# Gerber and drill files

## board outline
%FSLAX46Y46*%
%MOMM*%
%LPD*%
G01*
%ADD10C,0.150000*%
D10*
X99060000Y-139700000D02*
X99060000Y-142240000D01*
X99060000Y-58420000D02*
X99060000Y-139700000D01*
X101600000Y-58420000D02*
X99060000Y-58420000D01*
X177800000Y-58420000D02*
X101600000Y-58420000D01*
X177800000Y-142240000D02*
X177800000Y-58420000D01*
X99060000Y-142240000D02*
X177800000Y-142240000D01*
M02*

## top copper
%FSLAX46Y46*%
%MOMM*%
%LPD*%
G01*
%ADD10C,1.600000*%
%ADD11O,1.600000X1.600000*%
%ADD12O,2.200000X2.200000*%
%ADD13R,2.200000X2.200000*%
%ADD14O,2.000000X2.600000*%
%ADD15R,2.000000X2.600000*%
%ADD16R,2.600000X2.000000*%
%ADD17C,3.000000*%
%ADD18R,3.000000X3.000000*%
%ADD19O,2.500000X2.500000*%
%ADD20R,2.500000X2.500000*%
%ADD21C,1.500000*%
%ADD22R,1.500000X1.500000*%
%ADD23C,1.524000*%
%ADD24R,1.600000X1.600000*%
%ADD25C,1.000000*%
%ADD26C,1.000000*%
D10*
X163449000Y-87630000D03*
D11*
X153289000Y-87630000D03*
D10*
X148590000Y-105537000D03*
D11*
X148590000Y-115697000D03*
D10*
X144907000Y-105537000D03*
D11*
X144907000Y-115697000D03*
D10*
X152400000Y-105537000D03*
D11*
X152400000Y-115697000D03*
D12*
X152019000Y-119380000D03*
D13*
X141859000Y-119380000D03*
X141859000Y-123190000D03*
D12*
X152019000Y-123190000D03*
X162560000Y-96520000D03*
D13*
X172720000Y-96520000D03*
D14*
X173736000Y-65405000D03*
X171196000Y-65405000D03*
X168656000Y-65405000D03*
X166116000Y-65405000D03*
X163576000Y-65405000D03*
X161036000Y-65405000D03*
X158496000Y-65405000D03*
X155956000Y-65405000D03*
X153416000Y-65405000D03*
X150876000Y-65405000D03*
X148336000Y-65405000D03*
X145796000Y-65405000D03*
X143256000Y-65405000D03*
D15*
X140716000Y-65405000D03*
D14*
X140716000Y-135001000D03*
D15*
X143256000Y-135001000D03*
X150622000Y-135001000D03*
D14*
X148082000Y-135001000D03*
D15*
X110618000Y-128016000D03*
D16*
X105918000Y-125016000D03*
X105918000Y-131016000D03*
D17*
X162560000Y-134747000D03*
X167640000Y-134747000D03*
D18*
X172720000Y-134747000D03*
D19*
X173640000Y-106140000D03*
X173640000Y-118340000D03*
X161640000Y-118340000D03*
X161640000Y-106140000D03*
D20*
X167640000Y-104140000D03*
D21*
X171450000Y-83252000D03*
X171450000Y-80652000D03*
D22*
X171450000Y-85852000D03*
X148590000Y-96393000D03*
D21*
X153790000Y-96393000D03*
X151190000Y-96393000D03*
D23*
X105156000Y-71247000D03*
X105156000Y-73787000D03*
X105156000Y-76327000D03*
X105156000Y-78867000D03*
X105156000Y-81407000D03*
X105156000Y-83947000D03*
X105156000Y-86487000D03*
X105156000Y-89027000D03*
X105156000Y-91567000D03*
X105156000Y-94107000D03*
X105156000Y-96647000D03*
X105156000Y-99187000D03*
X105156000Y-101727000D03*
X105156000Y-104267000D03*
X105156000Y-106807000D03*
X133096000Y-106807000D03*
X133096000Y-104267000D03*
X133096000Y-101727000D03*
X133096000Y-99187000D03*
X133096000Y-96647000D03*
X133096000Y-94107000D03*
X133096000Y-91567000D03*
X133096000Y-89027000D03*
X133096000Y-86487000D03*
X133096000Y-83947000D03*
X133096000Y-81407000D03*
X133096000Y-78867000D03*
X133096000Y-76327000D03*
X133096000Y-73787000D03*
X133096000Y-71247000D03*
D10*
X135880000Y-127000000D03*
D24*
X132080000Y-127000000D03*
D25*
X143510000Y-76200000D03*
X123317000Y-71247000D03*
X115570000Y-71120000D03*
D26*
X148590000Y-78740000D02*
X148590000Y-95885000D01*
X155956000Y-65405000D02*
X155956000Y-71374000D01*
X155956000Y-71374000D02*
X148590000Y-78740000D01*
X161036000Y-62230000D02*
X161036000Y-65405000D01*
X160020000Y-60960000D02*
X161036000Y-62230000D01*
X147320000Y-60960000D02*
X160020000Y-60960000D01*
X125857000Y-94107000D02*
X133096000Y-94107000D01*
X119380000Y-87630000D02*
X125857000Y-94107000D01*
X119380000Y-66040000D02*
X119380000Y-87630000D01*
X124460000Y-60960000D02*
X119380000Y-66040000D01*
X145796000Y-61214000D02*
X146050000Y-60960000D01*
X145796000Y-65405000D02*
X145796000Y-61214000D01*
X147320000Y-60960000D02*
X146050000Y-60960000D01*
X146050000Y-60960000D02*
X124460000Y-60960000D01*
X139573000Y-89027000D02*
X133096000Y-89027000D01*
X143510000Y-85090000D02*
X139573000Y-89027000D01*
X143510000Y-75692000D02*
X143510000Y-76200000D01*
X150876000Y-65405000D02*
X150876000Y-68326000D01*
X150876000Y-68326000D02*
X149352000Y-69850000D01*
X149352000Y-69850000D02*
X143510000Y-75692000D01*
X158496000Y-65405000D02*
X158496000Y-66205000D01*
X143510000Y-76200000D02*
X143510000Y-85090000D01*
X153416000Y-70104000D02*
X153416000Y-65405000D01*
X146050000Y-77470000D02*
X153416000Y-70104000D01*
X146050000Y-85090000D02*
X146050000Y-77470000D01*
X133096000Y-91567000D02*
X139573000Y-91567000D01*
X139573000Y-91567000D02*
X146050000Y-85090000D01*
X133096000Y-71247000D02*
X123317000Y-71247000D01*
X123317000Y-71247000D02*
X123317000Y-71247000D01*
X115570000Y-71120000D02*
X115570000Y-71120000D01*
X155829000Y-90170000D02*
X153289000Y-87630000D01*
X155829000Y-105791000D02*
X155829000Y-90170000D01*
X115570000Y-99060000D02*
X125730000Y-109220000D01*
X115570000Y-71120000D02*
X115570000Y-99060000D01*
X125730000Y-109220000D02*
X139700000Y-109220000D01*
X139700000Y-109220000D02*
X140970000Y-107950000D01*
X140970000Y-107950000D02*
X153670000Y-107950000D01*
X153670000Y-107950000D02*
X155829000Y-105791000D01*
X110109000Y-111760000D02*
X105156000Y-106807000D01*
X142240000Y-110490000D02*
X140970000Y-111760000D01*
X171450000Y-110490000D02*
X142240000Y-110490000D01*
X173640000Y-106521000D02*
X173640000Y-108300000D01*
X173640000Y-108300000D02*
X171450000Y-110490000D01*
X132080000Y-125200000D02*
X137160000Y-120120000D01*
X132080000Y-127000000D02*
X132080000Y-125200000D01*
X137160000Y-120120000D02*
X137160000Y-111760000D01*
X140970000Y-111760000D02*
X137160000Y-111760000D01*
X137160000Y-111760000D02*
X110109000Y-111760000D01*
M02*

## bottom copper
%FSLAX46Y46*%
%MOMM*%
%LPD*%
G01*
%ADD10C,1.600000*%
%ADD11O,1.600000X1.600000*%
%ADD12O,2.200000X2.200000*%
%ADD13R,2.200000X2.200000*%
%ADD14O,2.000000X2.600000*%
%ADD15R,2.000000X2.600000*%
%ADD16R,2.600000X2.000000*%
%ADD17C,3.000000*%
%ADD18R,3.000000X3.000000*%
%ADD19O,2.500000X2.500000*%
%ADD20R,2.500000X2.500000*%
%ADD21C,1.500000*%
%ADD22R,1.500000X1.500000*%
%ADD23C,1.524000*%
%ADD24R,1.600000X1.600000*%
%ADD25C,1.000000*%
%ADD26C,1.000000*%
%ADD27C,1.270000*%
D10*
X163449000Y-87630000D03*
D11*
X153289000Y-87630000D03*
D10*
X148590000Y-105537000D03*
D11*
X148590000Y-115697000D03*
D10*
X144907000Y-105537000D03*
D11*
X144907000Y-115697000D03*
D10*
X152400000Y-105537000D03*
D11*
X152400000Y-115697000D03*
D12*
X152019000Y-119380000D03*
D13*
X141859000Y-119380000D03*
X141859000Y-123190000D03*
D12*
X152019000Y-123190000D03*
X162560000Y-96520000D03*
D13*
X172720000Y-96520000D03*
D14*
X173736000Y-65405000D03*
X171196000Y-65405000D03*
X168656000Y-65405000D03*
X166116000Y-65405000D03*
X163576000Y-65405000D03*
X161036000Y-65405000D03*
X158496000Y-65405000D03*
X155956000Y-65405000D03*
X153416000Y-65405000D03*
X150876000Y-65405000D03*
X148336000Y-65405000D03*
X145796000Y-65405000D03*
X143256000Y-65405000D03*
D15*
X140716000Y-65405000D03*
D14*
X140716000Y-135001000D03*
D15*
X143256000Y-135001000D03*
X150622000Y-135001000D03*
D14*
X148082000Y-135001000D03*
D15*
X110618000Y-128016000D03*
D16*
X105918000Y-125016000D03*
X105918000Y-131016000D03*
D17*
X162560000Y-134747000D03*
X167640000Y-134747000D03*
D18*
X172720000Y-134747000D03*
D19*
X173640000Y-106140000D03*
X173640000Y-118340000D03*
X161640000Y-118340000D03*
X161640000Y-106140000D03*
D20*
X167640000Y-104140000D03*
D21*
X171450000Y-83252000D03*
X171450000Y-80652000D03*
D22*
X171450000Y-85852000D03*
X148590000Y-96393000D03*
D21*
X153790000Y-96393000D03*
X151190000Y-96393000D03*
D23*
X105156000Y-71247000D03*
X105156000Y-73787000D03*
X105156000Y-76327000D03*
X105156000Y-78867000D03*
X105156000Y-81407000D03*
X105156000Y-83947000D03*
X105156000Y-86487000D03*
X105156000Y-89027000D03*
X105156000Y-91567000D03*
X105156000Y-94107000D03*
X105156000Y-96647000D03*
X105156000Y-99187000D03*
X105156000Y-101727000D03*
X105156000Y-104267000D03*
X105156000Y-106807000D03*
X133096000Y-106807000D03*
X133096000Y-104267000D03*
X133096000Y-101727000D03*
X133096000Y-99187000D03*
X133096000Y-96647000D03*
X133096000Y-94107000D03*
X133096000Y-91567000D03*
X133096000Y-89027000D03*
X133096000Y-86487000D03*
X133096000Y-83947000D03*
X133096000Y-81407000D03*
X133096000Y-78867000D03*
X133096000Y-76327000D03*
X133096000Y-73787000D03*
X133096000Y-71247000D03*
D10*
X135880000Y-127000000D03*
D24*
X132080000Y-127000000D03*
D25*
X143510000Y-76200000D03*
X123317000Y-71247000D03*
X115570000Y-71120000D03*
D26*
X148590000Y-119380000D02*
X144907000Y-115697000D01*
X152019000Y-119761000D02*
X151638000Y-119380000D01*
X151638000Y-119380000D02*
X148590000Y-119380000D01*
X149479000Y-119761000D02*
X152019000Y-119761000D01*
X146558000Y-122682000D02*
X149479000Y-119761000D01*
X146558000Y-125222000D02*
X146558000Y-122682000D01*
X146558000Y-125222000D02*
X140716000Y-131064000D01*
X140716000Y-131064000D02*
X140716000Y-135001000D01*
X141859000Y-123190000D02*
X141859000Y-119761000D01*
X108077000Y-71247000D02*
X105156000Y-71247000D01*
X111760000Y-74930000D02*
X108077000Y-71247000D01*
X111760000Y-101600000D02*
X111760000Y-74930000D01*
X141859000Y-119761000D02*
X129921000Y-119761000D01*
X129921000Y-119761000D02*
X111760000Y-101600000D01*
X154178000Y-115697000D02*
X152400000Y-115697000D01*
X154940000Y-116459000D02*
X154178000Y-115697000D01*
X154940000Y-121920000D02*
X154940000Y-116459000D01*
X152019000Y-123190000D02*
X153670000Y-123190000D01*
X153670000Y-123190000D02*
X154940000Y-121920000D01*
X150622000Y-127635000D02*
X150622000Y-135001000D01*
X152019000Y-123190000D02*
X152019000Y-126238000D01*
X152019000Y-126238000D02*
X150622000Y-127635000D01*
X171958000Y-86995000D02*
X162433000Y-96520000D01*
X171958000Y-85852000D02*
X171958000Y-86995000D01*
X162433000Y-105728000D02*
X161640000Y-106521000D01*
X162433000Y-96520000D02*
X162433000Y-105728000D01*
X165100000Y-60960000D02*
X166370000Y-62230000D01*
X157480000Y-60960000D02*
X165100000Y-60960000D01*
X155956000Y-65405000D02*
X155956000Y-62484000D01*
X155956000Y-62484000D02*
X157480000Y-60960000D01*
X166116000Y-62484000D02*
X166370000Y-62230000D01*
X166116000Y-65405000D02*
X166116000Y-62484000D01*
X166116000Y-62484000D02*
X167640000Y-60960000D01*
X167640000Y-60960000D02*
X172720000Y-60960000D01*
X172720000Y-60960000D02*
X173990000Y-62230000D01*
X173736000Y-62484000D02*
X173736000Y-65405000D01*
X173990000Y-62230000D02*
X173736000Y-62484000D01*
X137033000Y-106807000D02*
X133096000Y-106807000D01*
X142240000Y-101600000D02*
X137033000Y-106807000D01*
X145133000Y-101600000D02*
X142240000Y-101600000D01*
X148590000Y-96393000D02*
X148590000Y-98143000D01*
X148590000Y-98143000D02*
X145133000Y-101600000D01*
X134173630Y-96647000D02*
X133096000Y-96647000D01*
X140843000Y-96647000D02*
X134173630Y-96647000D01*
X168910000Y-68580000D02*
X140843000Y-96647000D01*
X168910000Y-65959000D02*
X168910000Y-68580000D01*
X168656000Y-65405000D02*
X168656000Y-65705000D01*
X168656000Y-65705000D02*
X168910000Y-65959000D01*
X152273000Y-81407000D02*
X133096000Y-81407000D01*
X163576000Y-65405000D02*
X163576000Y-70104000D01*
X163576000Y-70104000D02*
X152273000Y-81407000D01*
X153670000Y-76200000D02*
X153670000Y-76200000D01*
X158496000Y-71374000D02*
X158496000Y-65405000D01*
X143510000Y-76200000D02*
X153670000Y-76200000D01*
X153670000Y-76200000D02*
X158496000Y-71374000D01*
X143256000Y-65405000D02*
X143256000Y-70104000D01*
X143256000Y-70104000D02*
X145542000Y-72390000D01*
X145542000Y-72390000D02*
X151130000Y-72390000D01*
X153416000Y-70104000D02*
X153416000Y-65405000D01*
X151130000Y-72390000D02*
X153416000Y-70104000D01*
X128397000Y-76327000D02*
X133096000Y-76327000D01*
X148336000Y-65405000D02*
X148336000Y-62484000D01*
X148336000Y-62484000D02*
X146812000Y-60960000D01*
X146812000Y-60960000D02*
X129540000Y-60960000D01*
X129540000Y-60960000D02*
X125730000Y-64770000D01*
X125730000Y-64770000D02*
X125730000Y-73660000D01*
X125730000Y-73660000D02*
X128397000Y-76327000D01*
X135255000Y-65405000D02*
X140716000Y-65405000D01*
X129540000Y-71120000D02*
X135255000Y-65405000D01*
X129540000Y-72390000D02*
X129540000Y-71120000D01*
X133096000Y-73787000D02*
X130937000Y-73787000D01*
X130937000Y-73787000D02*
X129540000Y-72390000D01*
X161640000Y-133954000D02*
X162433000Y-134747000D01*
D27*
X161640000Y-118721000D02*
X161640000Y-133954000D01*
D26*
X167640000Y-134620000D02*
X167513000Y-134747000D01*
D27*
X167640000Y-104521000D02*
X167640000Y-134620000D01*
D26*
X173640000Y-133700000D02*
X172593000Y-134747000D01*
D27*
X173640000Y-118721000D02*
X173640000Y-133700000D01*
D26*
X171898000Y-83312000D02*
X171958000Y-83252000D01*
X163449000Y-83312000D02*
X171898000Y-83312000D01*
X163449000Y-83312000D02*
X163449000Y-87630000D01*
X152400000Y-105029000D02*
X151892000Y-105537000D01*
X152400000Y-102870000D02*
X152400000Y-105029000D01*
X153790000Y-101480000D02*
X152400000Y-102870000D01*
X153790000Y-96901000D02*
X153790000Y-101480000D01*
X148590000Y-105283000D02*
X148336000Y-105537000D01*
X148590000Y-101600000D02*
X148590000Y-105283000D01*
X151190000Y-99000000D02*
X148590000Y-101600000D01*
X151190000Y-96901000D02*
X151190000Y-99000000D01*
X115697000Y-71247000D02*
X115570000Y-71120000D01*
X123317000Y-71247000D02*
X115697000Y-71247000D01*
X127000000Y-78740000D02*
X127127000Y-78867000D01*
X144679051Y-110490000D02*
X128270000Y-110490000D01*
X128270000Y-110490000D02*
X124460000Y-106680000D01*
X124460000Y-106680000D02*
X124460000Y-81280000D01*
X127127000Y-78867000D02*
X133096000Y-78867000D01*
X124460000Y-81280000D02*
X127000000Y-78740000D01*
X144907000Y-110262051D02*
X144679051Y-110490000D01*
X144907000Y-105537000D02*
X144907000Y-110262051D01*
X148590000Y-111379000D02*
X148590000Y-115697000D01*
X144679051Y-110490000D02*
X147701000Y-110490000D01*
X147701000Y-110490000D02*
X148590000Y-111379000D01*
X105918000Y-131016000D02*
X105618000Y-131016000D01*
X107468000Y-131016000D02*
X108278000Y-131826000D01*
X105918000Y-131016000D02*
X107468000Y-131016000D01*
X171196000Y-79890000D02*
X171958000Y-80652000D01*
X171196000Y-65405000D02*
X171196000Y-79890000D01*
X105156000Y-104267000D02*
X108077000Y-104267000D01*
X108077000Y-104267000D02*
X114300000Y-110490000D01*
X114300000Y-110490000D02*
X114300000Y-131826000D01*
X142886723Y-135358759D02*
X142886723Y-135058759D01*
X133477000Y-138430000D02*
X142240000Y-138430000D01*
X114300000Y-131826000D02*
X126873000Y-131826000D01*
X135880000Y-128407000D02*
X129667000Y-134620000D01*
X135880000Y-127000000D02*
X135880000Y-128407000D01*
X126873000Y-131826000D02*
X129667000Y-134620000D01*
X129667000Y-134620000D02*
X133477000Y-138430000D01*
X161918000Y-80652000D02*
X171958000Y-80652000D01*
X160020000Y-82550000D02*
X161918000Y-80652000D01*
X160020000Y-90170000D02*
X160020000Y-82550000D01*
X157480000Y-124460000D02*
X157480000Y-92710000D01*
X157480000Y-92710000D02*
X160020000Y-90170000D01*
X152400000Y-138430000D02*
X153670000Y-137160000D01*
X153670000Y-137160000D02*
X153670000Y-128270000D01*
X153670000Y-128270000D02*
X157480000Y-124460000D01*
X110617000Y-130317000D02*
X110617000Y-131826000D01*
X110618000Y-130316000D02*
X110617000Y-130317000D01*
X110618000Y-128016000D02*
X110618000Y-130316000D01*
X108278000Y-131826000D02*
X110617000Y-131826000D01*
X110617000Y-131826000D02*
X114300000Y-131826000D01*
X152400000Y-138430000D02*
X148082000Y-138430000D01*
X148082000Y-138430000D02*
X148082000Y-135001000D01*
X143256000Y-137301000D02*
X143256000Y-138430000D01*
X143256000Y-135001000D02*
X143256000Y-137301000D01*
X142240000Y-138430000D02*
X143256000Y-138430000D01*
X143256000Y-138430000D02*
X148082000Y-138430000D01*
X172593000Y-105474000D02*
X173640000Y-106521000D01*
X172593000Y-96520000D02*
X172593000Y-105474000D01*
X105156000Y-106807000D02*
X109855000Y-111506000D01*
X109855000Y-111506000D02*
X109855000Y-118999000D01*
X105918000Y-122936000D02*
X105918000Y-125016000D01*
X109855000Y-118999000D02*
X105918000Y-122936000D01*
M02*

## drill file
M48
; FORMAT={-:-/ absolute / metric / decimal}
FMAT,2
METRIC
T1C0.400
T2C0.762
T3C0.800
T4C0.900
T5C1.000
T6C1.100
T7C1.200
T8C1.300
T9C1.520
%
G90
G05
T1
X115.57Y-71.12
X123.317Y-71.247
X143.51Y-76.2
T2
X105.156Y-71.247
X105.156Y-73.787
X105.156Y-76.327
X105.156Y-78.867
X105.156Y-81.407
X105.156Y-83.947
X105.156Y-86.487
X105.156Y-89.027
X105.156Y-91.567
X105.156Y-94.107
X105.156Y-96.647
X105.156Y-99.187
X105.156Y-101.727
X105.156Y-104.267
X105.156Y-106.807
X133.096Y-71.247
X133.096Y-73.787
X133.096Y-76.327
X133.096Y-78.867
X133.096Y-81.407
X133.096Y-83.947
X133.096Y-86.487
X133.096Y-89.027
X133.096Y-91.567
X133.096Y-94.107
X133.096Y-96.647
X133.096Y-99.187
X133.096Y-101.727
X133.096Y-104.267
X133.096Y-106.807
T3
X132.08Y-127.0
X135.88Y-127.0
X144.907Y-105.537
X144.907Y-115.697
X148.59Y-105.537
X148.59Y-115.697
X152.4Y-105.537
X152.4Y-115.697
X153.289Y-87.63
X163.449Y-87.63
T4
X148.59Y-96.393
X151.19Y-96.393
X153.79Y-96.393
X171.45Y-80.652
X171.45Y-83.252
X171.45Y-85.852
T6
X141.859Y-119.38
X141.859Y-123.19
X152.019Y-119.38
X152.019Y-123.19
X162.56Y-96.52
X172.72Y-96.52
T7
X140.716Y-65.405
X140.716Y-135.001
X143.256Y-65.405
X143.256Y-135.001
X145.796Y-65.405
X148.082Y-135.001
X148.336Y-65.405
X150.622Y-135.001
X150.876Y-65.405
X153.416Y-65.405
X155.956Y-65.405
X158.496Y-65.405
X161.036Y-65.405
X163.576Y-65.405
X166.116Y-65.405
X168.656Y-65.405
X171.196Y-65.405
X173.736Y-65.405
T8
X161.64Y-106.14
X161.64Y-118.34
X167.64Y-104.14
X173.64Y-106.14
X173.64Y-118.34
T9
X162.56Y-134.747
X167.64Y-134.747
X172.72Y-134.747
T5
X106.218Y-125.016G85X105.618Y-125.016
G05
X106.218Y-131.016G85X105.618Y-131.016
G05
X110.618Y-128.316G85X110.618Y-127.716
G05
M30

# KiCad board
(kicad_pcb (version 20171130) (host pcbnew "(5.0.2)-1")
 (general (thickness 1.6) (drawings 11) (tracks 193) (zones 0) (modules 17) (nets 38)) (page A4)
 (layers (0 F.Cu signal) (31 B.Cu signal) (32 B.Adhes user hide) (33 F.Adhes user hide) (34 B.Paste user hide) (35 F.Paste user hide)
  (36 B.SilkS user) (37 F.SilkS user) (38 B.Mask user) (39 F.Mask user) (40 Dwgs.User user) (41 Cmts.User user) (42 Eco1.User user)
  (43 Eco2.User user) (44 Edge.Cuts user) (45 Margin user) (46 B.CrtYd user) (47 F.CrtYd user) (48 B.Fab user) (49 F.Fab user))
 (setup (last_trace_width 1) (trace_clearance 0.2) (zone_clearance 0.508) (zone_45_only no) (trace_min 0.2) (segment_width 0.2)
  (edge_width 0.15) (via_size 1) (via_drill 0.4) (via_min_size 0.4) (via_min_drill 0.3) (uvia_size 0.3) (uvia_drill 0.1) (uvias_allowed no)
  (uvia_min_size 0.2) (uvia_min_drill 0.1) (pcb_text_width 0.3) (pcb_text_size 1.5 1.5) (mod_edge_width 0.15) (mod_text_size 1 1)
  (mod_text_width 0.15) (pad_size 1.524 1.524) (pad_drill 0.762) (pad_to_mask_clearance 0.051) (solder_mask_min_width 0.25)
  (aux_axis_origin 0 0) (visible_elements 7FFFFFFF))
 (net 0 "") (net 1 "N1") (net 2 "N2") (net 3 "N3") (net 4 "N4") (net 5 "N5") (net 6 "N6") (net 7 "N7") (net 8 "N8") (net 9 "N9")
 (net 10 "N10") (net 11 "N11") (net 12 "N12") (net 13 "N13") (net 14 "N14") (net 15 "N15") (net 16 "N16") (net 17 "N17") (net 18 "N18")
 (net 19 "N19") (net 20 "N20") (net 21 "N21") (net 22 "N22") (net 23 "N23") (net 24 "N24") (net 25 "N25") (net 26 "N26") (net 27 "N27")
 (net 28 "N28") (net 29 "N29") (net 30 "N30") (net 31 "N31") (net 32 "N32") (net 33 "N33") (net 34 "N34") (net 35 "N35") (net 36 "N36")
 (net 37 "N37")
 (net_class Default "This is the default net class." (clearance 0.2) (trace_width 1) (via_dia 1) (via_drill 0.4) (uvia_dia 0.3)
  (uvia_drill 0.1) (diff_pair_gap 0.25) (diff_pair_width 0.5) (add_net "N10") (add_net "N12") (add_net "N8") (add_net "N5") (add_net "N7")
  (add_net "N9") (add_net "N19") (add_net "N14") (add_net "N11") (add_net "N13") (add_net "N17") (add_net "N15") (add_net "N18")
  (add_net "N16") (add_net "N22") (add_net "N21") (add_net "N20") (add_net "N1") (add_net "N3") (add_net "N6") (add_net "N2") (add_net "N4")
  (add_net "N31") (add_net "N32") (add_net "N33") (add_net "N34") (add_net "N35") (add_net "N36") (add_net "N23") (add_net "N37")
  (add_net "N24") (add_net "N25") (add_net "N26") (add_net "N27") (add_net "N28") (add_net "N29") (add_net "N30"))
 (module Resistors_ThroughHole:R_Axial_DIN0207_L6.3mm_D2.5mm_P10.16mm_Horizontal (layer F.Cu) (at 163.449 87.63 180)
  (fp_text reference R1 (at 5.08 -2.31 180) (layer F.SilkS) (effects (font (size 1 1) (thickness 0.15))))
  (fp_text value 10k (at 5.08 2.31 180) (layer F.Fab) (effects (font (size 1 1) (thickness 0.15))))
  (pad 1 thru_hole circle (at 0 0 180) (size 1.6 1.6) (drill 0.8) (layers *.Cu *.Mask) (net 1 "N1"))
  (pad 2 thru_hole oval (at 10.16 0 180) (size 1.6 1.6) (drill 0.8) (layers *.Cu *.Mask) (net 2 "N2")))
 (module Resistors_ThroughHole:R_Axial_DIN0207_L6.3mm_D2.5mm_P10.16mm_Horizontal (layer F.Cu) (at 148.59 105.537 270)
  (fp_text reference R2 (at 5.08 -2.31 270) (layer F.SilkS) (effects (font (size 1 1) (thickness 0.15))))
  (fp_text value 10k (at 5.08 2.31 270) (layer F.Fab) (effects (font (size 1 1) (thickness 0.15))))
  (pad 1 thru_hole circle (at 0 0 270) (size 1.6 1.6) (drill 0.8) (layers *.Cu *.Mask) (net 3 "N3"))
  (pad 2 thru_hole oval (at 10.16 0 270) (size 1.6 1.6) (drill 0.8) (layers *.Cu *.Mask) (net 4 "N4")))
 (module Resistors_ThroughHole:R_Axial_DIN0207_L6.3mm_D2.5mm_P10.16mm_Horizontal (layer F.Cu) (at 144.907 105.537 270)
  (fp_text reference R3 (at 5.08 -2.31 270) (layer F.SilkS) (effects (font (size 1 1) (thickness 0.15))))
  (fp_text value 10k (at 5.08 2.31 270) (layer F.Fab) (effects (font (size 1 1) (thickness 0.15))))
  (pad 1 thru_hole circle (at 0 0 270) (size 1.6 1.6) (drill 0.8) (layers *.Cu *.Mask) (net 4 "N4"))
  (pad 2 thru_hole oval (at 10.16 0 270) (size 1.6 1.6) (drill 0.8) (layers *.Cu *.Mask) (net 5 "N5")))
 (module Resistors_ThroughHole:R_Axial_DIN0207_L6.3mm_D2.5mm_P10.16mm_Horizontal (layer F.Cu) (at 152.4 105.537 270)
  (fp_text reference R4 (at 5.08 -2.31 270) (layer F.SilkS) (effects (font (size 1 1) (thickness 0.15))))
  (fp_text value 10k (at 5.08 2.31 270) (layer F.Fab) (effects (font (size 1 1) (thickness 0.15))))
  (pad 1 thru_hole circle (at 0 0 270) (size 1.6 1.6) (drill 0.8) (layers *.Cu *.Mask) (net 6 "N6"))
  (pad 2 thru_hole oval (at 10.16 0 270) (size 1.6 1.6) (drill 0.8) (layers *.Cu *.Mask) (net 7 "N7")))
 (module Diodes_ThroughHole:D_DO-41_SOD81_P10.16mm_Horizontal (layer F.Cu) (at 141.859 119.38)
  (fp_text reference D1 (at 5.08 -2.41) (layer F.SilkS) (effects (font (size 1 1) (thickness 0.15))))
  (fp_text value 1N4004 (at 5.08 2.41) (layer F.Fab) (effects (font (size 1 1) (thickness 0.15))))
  (pad 2 thru_hole oval (at 10.16 0) (size 2.2 2.2) (drill 1.1) (layers *.Cu *.Mask) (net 5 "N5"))
  (pad 1 thru_hole rect (at 0 0) (size 2.2 2.2) (drill 1.1) (layers *.Cu *.Mask) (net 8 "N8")))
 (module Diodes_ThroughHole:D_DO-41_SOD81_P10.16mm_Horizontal (layer F.Cu) (at 141.859 123.19)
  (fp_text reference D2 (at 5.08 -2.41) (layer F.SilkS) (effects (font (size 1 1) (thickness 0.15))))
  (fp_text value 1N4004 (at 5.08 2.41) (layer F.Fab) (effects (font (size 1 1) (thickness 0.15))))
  (pad 1 thru_hole rect (at 0 0) (size 2.2 2.2) (drill 1.1) (layers *.Cu *.Mask) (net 8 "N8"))
  (pad 2 thru_hole oval (at 10.16 0) (size 2.2 2.2) (drill 1.1) (layers *.Cu *.Mask) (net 7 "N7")))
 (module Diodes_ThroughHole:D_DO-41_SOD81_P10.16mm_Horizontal (layer F.Cu) (at 172.72 96.52 180)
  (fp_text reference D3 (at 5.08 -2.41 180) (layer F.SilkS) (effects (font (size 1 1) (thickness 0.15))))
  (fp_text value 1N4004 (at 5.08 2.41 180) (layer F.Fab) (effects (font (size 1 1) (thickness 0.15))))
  (pad 2 thru_hole oval (at 10.16 0 180) (size 2.2 2.2) (drill 1.1) (layers *.Cu *.Mask) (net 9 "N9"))
  (pad 1 thru_hole rect (at 0 0 180) (size 2.2 2.2) (drill 1.1) (layers *.Cu *.Mask) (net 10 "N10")))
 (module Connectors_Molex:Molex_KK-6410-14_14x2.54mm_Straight (layer F.Cu) (at 140.716 65.405)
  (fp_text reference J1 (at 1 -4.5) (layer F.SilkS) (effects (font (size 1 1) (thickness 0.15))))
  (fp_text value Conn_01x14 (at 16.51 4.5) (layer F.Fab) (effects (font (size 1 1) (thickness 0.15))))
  (pad 14 thru_hole oval (at 33.02 0) (size 2 2.6) (drill 1.2) (layers *.Cu *.Mask) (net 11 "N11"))
  (pad 13 thru_hole oval (at 30.48 0) (size 2 2.6) (drill 1.2) (layers *.Cu *.Mask) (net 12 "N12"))
  (pad 12 thru_hole oval (at 27.94 0) (size 2 2.6) (drill 1.2) (layers *.Cu *.Mask) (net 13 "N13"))
  (pad 11 thru_hole oval (at 25.4 0) (size 2 2.6) (drill 1.2) (layers *.Cu *.Mask) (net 11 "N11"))
  (pad 10 thru_hole oval (at 22.86 0) (size 2 2.6) (drill 1.2) (layers *.Cu *.Mask) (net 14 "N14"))
  (pad 9 thru_hole oval (at 20.32 0) (size 2 2.6) (drill 1.2) (layers *.Cu *.Mask) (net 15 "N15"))
  (pad 8 thru_hole oval (at 17.78 0) (size 2 2.6) (drill 1.2) (layers *.Cu *.Mask) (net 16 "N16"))
  (pad 7 thru_hole oval (at 15.24 0) (size 2 2.6) (drill 1.2) (layers *.Cu *.Mask) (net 11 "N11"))
  (pad 6 thru_hole oval (at 12.7 0) (size 2 2.6) (drill 1.2) (layers *.Cu *.Mask) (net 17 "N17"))
  (pad 5 thru_hole oval (at 10.16 0) (size 2 2.6) (drill 1.2) (layers *.Cu *.Mask) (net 16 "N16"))
  (pad 4 thru_hole oval (at 7.62 0) (size 2 2.6) (drill 1.2) (layers *.Cu *.Mask) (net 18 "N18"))
  (pad 3 thru_hole oval (at 5.08 0) (size 2 2.6) (drill 1.2) (layers *.Cu *.Mask) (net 15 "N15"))
  (pad 2 thru_hole oval (at 2.54 0) (size 2 2.6) (drill 1.2) (layers *.Cu *.Mask) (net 17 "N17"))
  (pad 1 thru_hole rect (at 0 0) (size 2 2.6) (drill 1.2) (layers *.Cu *.Mask) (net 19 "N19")))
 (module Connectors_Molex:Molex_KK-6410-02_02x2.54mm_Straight (layer F.Cu) (at 143.256 135.001 180)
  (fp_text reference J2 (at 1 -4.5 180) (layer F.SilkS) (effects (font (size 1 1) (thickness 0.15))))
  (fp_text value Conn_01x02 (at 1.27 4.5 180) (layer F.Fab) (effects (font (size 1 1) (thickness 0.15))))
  (pad 2 thru_hole oval (at 2.54 0 180) (size 2 2.6) (drill 1.2) (layers *.Cu *.Mask) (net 5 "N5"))
  (pad 1 thru_hole rect (at 0 0 180) (size 2 2.6) (drill 1.2) (layers *.Cu *.Mask) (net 12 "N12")))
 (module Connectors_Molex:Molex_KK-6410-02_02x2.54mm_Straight (layer F.Cu) (at 150.622 135.001 180)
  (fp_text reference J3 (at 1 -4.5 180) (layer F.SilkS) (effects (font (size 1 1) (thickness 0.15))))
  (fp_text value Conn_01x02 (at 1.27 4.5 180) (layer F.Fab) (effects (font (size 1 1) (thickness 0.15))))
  (pad 1 thru_hole rect (at 0 0 180) (size 2 2.6) (drill 1.2) (layers *.Cu *.Mask) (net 7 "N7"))
  (pad 2 thru_hole oval (at 2.54 0 180) (size 2 2.6) (drill 1.2) (layers *.Cu *.Mask) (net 12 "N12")))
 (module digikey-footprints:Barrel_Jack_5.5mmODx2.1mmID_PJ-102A (layer F.Cu) (at 105.918 128.016 180)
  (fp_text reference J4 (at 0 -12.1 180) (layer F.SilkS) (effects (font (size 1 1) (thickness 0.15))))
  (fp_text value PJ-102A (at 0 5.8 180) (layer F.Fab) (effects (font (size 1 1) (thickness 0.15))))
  (pad 3 thru_hole rect (at -4.7 0 180) (size 2 2.6) (drill oval 1 1.6) (layers *.Cu *.Mask) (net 12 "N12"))
  (pad 1 thru_hole rect (at 0 3 180) (size 2.6 2) (drill oval 1.6 1) (layers *.Cu *.Mask) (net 10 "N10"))
  (pad 2 thru_hole rect (at 0 -3 180) (size 2.6 2) (drill oval 1.6 1) (layers *.Cu *.Mask) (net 12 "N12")))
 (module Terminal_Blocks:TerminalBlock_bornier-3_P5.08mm (layer F.Cu) (at 172.72 134.747 180)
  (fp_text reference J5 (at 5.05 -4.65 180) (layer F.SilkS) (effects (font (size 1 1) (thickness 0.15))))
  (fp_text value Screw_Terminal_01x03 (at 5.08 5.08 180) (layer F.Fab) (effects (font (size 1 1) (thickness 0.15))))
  (pad 3 thru_hole circle (at 10.16 0 180) (size 3 3) (drill 1.52) (layers *.Cu *.Mask) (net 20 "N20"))
  (pad 2 thru_hole circle (at 5.08 0 180) (size 3 3) (drill 1.52) (layers *.Cu *.Mask) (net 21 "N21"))
  (pad 1 thru_hole rect (at 0 0 180) (size 3 3) (drill 1.52) (layers *.Cu *.Mask) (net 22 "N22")))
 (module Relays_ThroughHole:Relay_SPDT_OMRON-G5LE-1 (layer F.Cu) (at 167.64 104.14)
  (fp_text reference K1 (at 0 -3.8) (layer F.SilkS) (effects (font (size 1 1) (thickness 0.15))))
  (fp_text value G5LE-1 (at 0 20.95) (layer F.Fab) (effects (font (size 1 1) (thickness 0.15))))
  (pad 5 thru_hole oval (at 6 2) (size 2.5 2.5) (drill 1.3) (layers *.Cu *.Mask) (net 10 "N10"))
  (pad 4 thru_hole oval (at 6 14.2) (size 2.5 2.5) (drill 1.3) (layers *.Cu *.Mask) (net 22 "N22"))
  (pad 3 thru_hole oval (at -6 14.2) (size 2.5 2.5) (drill 1.3) (layers *.Cu *.Mask) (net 20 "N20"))
  (pad 2 thru_hole oval (at -6 2) (size 2.5 2.5) (drill 1.3) (layers *.Cu *.Mask) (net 9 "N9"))
  (pad 1 thru_hole rect (at 0 0) (size 2.5 2.5) (drill 1.3) (layers *.Cu *.Mask) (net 21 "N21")))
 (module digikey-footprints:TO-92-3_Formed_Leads (layer F.Cu) (at 171.45 85.852 90)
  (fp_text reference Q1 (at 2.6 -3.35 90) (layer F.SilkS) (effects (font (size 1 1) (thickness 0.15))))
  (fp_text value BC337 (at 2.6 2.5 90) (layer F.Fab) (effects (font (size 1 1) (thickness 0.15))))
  (pad 2 thru_hole circle (at 2.6 0 270) (size 1.5 1.5) (drill 0.9) (layers *.Cu *.Mask) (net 1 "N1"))
  (pad 3 thru_hole circle (at 5.2 0 270) (size 1.5 1.5) (drill 0.9) (layers *.Cu *.Mask) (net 12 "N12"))
  (pad 1 thru_hole rect (at 0 0 270) (size 1.5 1.5) (drill 0.9) (layers *.Cu *.Mask) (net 9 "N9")))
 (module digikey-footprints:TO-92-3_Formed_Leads (layer F.Cu) (at 148.59 96.393)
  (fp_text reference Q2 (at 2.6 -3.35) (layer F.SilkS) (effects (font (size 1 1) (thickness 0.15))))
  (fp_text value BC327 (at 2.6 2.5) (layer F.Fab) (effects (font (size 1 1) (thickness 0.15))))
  (pad 1 thru_hole rect (at 0 0 180) (size 1.5 1.5) (drill 0.9) (layers *.Cu *.Mask) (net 11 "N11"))
  (pad 3 thru_hole circle (at 5.2 0 180) (size 1.5 1.5) (drill 0.9) (layers *.Cu *.Mask) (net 6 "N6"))
  (pad 2 thru_hole circle (at 2.6 0 180) (size 1.5 1.5) (drill 0.9) (layers *.Cu *.Mask) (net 3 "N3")))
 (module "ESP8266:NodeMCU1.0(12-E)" (layer F.Cu) (at 119.126 92.202)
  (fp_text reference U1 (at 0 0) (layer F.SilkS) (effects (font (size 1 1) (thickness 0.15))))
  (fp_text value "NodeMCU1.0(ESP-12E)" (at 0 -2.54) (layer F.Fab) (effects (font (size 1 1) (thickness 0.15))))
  (pad 1 thru_hole circle (at -13.97 -20.955) (size 1.524 1.524) (drill 0.762) (layers *.Cu *.Mask F.SilkS) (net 8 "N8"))
  (pad 2 thru_hole circle (at -13.97 -18.415) (size 1.524 1.524) (drill 0.762) (layers *.Cu *.Mask F.SilkS) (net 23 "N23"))
  (pad 3 thru_hole circle (at -13.97 -15.875) (size 1.524 1.524) (drill 0.762) (layers *.Cu *.Mask F.SilkS) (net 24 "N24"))
  (pad 4 thru_hole circle (at -13.97 -13.335) (size 1.524 1.524) (drill 0.762) (layers *.Cu *.Mask F.SilkS) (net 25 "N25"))
  (pad 5 thru_hole circle (at -13.97 -10.795) (size 1.524 1.524) (drill 0.762) (layers *.Cu *.Mask F.SilkS) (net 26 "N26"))
  (pad 6 thru_hole circle (at -13.97 -8.255) (size 1.524 1.524) (drill 0.762) (layers *.Cu *.Mask F.SilkS) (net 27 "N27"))
  (pad 7 thru_hole circle (at -13.97 -5.715) (size 1.524 1.524) (drill 0.762) (layers *.Cu *.Mask F.SilkS) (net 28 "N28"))
  (pad 8 thru_hole circle (at -13.97 -3.175) (size 1.524 1.524) (drill 0.762) (layers *.Cu *.Mask F.SilkS) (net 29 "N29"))
  (pad 9 thru_hole circle (at -13.97 -0.635) (size 1.524 1.524) (drill 0.762) (layers *.Cu *.Mask F.SilkS) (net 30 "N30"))
  (pad 10 thru_hole circle (at -13.97 1.905) (size 1.524 1.524) (drill 0.762) (layers *.Cu *.Mask F.SilkS) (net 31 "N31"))
  (pad 11 thru_hole circle (at -13.97 4.445) (size 1.524 1.524) (drill 0.762) (layers *.Cu *.Mask F.SilkS) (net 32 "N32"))
  (pad 12 thru_hole circle (at -13.97 6.985) (size 1.524 1.524) (drill 0.762) (layers *.Cu *.Mask F.SilkS) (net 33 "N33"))
  (pad 13 thru_hole circle (at -13.97 9.525) (size 1.524 1.524) (drill 0.762) (layers *.Cu *.Mask F.SilkS) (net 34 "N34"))
  (pad 14 thru_hole circle (at -13.97 12.065) (size 1.524 1.524) (drill 0.762) (layers *.Cu *.Mask F.SilkS) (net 12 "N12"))
  (pad 15 thru_hole circle (at -13.97 14.605) (size 1.524 1.524) (drill 0.762) (layers *.Cu *.Mask F.SilkS) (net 10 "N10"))
  (pad 16 thru_hole circle (at 13.97 14.605) (size 1.524 1.524) (drill 0.762) (layers *.Cu *.Mask F.SilkS) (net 11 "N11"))
  (pad 17 thru_hole circle (at 13.97 12.065) (size 1.524 1.524) (drill 0.762) (layers *.Cu *.Mask F.SilkS) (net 12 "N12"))
  (pad 18 thru_hole circle (at 13.97 9.525) (size 1.524 1.524) (drill 0.762) (layers *.Cu *.Mask F.SilkS) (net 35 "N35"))
  (pad 19 thru_hole circle (at 13.97 6.985) (size 1.524 1.524) (drill 0.762) (layers *.Cu *.Mask F.SilkS) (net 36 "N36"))
  (pad 20 thru_hole circle (at 13.97 4.445) (size 1.524 1.524) (drill 0.762) (layers *.Cu *.Mask F.SilkS) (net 13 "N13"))
  (pad 21 thru_hole circle (at 13.97 1.905) (size 1.524 1.524) (drill 0.762) (layers *.Cu *.Mask F.SilkS) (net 15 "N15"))
  (pad 22 thru_hole circle (at 13.97 -0.635) (size 1.524 1.524) (drill 0.762) (layers *.Cu *.Mask F.SilkS) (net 17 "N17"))
  (pad 23 thru_hole circle (at 13.97 -3.175) (size 1.524 1.524) (drill 0.762) (layers *.Cu *.Mask F.SilkS) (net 16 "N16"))
  (pad 24 thru_hole circle (at 13.97 -5.715) (size 1.524 1.524) (drill 0.762) (layers *.Cu *.Mask F.SilkS) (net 12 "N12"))
  (pad 25 thru_hole circle (at 13.97 -8.255) (size 1.524 1.524) (drill 0.762) (layers *.Cu *.Mask F.SilkS) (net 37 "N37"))
  (pad 26 thru_hole circle (at 13.97 -10.795) (size 1.524 1.524) (drill 0.762) (layers *.Cu *.Mask F.SilkS) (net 14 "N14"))
  (pad 27 thru_hole circle (at 13.97 -13.335) (size 1.524 1.524) (drill 0.762) (layers *.Cu *.Mask F.SilkS) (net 4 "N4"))
  (pad 28 thru_hole circle (at 13.97 -15.875) (size 1.524 1.524) (drill 0.762) (layers *.Cu *.Mask F.SilkS) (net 18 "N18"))
  (pad 29 thru_hole circle (at 13.97 -18.415) (size 1.524 1.524) (drill 0.762) (layers *.Cu *.Mask F.SilkS) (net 19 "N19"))
  (pad 30 thru_hole circle (at 13.97 -20.955) (size 1.524 1.524) (drill 0.762) (layers *.Cu *.Mask F.SilkS) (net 2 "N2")))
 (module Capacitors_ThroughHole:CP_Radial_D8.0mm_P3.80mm (layer F.Cu) (at 132.08 127)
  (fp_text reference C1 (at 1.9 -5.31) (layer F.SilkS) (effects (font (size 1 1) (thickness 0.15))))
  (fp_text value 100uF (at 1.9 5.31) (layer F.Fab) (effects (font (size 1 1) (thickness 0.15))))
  (pad 2 thru_hole circle (at 3.8 0) (size 1.6 1.6) (drill 0.8) (layers *.Cu *.Mask) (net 12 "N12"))
  (pad 1 thru_hole rect (at 0 0) (size 1.6 1.6) (drill 0.8) (layers *.Cu *.Mask) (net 10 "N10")))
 (gr_line (start 99.06 139.7) (end 99.06 142.24) (layer Edge.Cuts) (width 0.15))
 (gr_line (start 99.06 58.42) (end 99.06 139.7) (layer Edge.Cuts) (width 0.15))
 (gr_line (start 101.6 58.42) (end 99.06 58.42) (layer Edge.Cuts) (width 0.15))
 (gr_line (start 177.8 58.42) (end 101.6 58.42) (layer Edge.Cuts) (width 0.15))
 (gr_line (start 177.8 142.24) (end 177.8 58.42) (layer Edge.Cuts) (width 0.15))
 (gr_line (start 99.06 142.24) (end 177.8 142.24) (layer Edge.Cuts) (width 0.15))
 (segment (start 148.59 119.38) (end 144.907 115.697) (width 1) (layer B.Cu) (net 5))
 (segment (start 152.019 119.761) (end 151.638 119.38) (width 1) (layer B.Cu) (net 5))
 (segment (start 151.638 119.38) (end 148.59 119.38) (width 1) (layer B.Cu) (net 5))
 (segment (start 149.479 119.761) (end 152.019 119.761) (width 1) (layer B.Cu) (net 5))
 (segment (start 146.558 122.682) (end 149.479 119.761) (width 1) (layer B.Cu) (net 5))
 (segment (start 146.558 125.222) (end 146.558 122.682) (width 1) (layer B.Cu) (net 5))
 (segment (start 146.558 125.222) (end 140.716 131.064) (width 1) (layer B.Cu) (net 5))
 (segment (start 140.716 131.064) (end 140.716 135.001) (width 1) (layer B.Cu) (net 5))
 (segment (start 141.859 123.19) (end 141.859 119.761) (width 1) (layer B.Cu) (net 8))
 (segment (start 108.077 71.247) (end 105.156 71.247) (width 1) (layer B.Cu) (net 8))
 (segment (start 111.76 74.93) (end 108.077 71.247) (width 1) (layer B.Cu) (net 8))
 (segment (start 111.76 101.6) (end 111.76 74.93) (width 1) (layer B.Cu) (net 8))
 (segment (start 141.859 119.761) (end 129.921 119.761) (width 1) (layer B.Cu) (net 8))
 (segment (start 129.921 119.761) (end 111.76 101.6) (width 1) (layer B.Cu) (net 8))
 (segment (start 154.178 115.697) (end 152.4 115.697) (width 1) (layer B.Cu) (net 7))
 (segment (start 154.94 116.459) (end 154.178 115.697) (width 1) (layer B.Cu) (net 7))
 (segment (start 154.94 121.92) (end 154.94 116.459) (width 1) (layer B.Cu) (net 7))
 (segment (start 152.019 123.19) (end 153.67 123.19) (width 1) (layer B.Cu) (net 7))
 (segment (start 153.67 123.19) (end 154.94 121.92) (width 1) (layer B.Cu) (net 7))
 (segment (start 150.622 127.635) (end 150.622 135.001) (width 1) (layer B.Cu) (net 7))
 (segment (start 152.019 123.19) (end 152.019 126.238) (width 1) (layer B.Cu) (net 7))
 (segment (start 152.019 126.238) (end 150.622 127.635) (width 1) (layer B.Cu) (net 7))
 (segment (start 171.958 86.995) (end 162.433 96.52) (width 1) (layer B.Cu) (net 9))
 (segment (start 171.958 85.852) (end 171.958 86.995) (width 1) (layer B.Cu) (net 9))
 (segment (start 162.433 105.728) (end 161.64 106.521) (width 1) (layer B.Cu) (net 9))
 (segment (start 162.433 96.52) (end 162.433 105.728) (width 1) (layer B.Cu) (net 9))
 (segment (start 165.1 60.96) (end 166.37 62.23) (width 1) (layer B.Cu) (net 11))
 (segment (start 157.48 60.96) (end 165.1 60.96) (width 1) (layer B.Cu) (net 11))
 (segment (start 155.956 65.405) (end 155.956 62.484) (width 1) (layer B.Cu) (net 11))
 (segment (start 155.956 62.484) (end 157.48 60.96) (width 1) (layer B.Cu) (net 11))
 (segment (start 166.116 62.484) (end 166.37 62.23) (width 1) (layer B.Cu) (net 11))
 (segment (start 166.116 65.405) (end 166.116 62.484) (width 1) (layer B.Cu) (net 11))
 (segment (start 166.116 62.484) (end 167.64 60.96) (width 1) (layer B.Cu) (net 11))
 (segment (start 167.64 60.96) (end 172.72 60.96) (width 1) (layer B.Cu) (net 11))
 (segment (start 172.72 60.96) (end 173.99 62.23) (width 1) (layer B.Cu) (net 11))
 (segment (start 173.736 62.484) (end 173.736 65.405) (width 1) (layer B.Cu) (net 11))
 (segment (start 173.99 62.23) (end 173.736 62.484) (width 1) (layer B.Cu) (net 11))
 (segment (start 148.59 78.74) (end 148.59 95.885) (width 1) (layer F.Cu) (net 11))
 (segment (start 155.956 65.405) (end 155.956 71.374) (width 1) (layer F.Cu) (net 11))
 (segment (start 155.956 71.374) (end 148.59 78.74) (width 1) (layer F.Cu) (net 11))
 (segment (start 137.033 106.807) (end 133.096 106.807) (width 1) (layer B.Cu) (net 11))
 (segment (start 142.24 101.6) (end 137.033 106.807) (width 1) (layer B.Cu) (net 11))
 (segment (start 145.133 101.6) (end 142.24 101.6) (width 1) (layer B.Cu) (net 11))
 (segment (start 148.59 96.393) (end 148.59 98.143) (width 1) (layer B.Cu) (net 11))
 (segment (start 148.59 98.143) (end 145.133 101.6) (width 1) (layer B.Cu) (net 11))
 (segment (start 134.17363 96.647) (end 133.096 96.647) (width 1) (layer B.Cu) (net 13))
 (segment (start 140.843 96.647) (end 134.17363 96.647) (width 1) (layer B.Cu) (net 13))
 (segment (start 168.91 68.58) (end 140.843 96.647) (width 1) (layer B.Cu) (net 13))
 (segment (start 168.91 65.959) (end 168.91 68.58) (width 1) (layer B.Cu) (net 13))
 (segment (start 168.656 65.405) (end 168.656 65.705) (width 1) (layer B.Cu) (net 13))
 (segment (start 168.656 65.705) (end 168.91 65.959) (width 1) (layer B.Cu) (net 13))
 (segment (start 152.273 81.407) (end 133.096 81.407) (width 1) (layer B.Cu) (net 14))
 (segment (start 163.576 65.405) (end 163.576 70.104) (width 1) (layer B.Cu) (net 14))
 (segment (start 163.576 70.104) (end 152.273 81.407) (width 1) (layer B.Cu) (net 14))
 (segment (start 161.036 62.23) (end 161.036 65.405) (width 1) (layer F.Cu) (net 15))
 (segment (start 160.02 60.96) (end 161.036 62.23) (width 1) (layer F.Cu) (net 15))
 (segment (start 147.32 60.96) (end 160.02 60.96) (width 1) (layer F.Cu) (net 15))
 (segment (start 125.857 94.107) (end 133.096 94.107) (width 1) (layer F.Cu) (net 15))
 (segment (start 119.38 87.63) (end 125.857 94.107) (width 1) (layer F.Cu) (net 15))
 (segment (start 119.38 66.04) (end 119.38 87.63) (width 1) (layer F.Cu) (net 15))
 (segment (start 124.46 60.96) (end 119.38 66.04) (width 1) (layer F.Cu) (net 15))
 (segment (start 145.796 61.214) (end 146.05 60.96) (width 1) (layer F.Cu) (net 15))
 (segment (start 145.796 65.405) (end 145.796 61.214) (width 1) (layer F.Cu) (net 15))
 (segment (start 147.32 60.96) (end 146.05 60.96) (width 1) (layer F.Cu) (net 15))
 (segment (start 146.05 60.96) (end 124.46 60.96) (width 1) (layer F.Cu) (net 15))
 (segment (start 139.573 89.027) (end 133.096 89.027) (width 1) (layer F.Cu) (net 16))
 (segment (start 143.51 85.09) (end 139.573 89.027) (width 1) (layer F.Cu) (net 16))
 (segment (start 143.51 75.692) (end 143.51 76.2) (width 1) (layer F.Cu) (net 16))
 (segment (start 150.876 65.405) (end 150.876 68.326) (width 1) (layer F.Cu) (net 16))
 (segment (start 150.876 68.326) (end 149.352 69.85) (width 1) (layer F.Cu) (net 16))
 (segment (start 149.352 69.85) (end 143.51 75.692) (width 1) (layer F.Cu) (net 16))
 (segment (start 158.496 65.405) (end 158.496 66.205) (width 1) (layer F.Cu) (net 16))
 (segment (start 143.51 76.2) (end 143.51 85.09) (width 1) (layer F.Cu) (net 16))
 (via (at 143.51 76.2) (size 1) (drill 0.4) (layers F.Cu B.Cu) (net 16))
 (segment (start 153.67 76.2) (end 153.67 76.2) (width 1) (layer B.Cu) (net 16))
 (segment (start 158.496 71.374) (end 158.496 65.405) (width 1) (layer B.Cu) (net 16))
 (segment (start 143.51 76.2) (end 153.67 76.2) (width 1) (layer B.Cu) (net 16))
 (segment (start 153.67 76.2) (end 158.496 71.374) (width 1) (layer B.Cu) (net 16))
 (segment (start 143.256 65.405) (end 143.256 70.104) (width 1) (layer B.Cu) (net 17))
 (segment (start 143.256 70.104) (end 145.542 72.39) (width 1) (layer B.Cu) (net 17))
 (segment (start 145.542 72.39) (end 151.13 72.39) (width 1) (layer B.Cu) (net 17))
 (segment (start 153.416 70.104) (end 153.416 65.405) (width 1) (layer B.Cu) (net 17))
 (segment (start 151.13 72.39) (end 153.416 70.104) (width 1) (layer B.Cu) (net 17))
 (segment (start 153.416 70.104) (end 153.416 65.405) (width 1) (layer F.Cu) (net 17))
 (segment (start 146.05 77.47) (end 153.416 70.104) (width 1) (layer F.Cu) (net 17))
 (segment (start 146.05 85.09) (end 146.05 77.47) (width 1) (layer F.Cu) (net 17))
 (segment (start 133.096 91.567) (end 139.573 91.567) (width 1) (layer F.Cu) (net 17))
 (segment (start 139.573 91.567) (end 146.05 85.09) (width 1) (layer F.Cu) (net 17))
 (segment (start 128.397 76.327) (end 133.096 76.327) (width 1) (layer B.Cu) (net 18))
 (segment (start 148.336 65.405) (end 148.336 62.484) (width 1) (layer B.Cu) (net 18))
 (segment (start 148.336 62.484) (end 146.812 60.96) (width 1) (layer B.Cu) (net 18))
 (segment (start 146.812 60.96) (end 129.54 60.96) (width 1) (layer B.Cu) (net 18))
 (segment (start 129.54 60.96) (end 125.73 64.77) (width 1) (layer B.Cu) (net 18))
 (segment (start 125.73 64.77) (end 125.73 73.66) (width 1) (layer B.Cu) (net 18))
 (segment (start 125.73 73.66) (end 128.397 76.327) (width 1) (layer B.Cu) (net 18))
 (segment (start 135.255 65.405) (end 140.716 65.405) (width 1) (layer B.Cu) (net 19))
 (segment (start 129.54 71.12) (end 135.255 65.405) (width 1) (layer B.Cu) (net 19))
 (segment (start 129.54 72.39) (end 129.54 71.12) (width 1) (layer B.Cu) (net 19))
 (segment (start 133.096 73.787) (end 130.937 73.787) (width 1) (layer B.Cu) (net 19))
 (segment (start 130.937 73.787) (end 129.54 72.39) (width 1) (layer B.Cu) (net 19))
 (segment (start 161.64 133.954) (end 162.433 134.747) (width 1) (layer B.Cu) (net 20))
 (segment (start 161.64 118.721) (end 161.64 133.954) (width 1.27) (layer B.Cu) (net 20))
 (segment (start 167.64 134.62) (end 167.513 134.747) (width 1) (layer B.Cu) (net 21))
 (segment (start 167.64 104.521) (end 167.64 134.62) (width 1.27) (layer B.Cu) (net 21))
 (segment (start 173.64 133.7) (end 172.593 134.747) (width 1) (layer B.Cu) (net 22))
 (segment (start 173.64 118.721) (end 173.64 133.7) (width 1.27) (layer B.Cu) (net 22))
 (segment (start 171.898 83.312) (end 171.958 83.252) (width 1) (layer B.Cu) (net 1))
 (segment (start 163.449 83.312) (end 171.898 83.312) (width 1) (layer B.Cu) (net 1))
 (segment (start 163.449 83.312) (end 163.449 87.63) (width 1) (layer B.Cu) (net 1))
 (segment (start 152.4 105.029) (end 151.892 105.537) (width 1) (layer B.Cu) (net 6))
 (segment (start 152.4 102.87) (end 152.4 105.029) (width 1) (layer B.Cu) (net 6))
 (segment (start 153.79 101.48) (end 152.4 102.87) (width 1) (layer B.Cu) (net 6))
 (segment (start 153.79 96.901) (end 153.79 101.48) (width 1) (layer B.Cu) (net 6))
 (segment (start 148.59 105.283) (end 148.336 105.537) (width 1) (layer B.Cu) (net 3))
 (segment (start 148.59 101.6) (end 148.59 105.283) (width 1) (layer B.Cu) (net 3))
 (segment (start 151.19 99) (end 148.59 101.6) (width 1) (layer B.Cu) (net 3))
 (segment (start 151.19 96.901) (end 151.19 99) (width 1) (layer B.Cu) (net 3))
 (segment (start 133.096 71.247) (end 123.317 71.247) (width 1) (layer F.Cu) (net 2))
 (segment (start 123.317 71.247) (end 123.317 71.247) (width 1) (layer F.Cu) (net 2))
 (via (at 123.317 71.247) (size 1) (drill 0.4) (layers F.Cu B.Cu) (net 2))
 (segment (start 115.57 71.12) (end 115.57 71.12) (width 1) (layer F.Cu) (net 2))
 (via (at 115.57 71.12) (size 1) (drill 0.4) (layers F.Cu B.Cu) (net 2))
 (segment (start 115.697 71.247) (end 115.57 71.12) (width 1) (layer B.Cu) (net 2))
 (segment (start 123.317 71.247) (end 115.697 71.247) (width 1) (layer B.Cu) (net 2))
 (segment (start 155.829 90.17) (end 153.289 87.63) (width 1) (layer F.Cu) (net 2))
 (segment (start 155.829 105.791) (end 155.829 90.17) (width 1) (layer F.Cu) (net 2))
 (segment (start 115.57 99.06) (end 125.73 109.22) (width 1) (layer F.Cu) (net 2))
 (segment (start 115.57 71.12) (end 115.57 99.06) (width 1) (layer F.Cu) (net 2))
 (segment (start 125.73 109.22) (end 139.7 109.22) (width 1) (layer F.Cu) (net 2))
 (segment (start 139.7 109.22) (end 140.97 107.95) (width 1) (layer F.Cu) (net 2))
 (segment (start 140.97 107.95) (end 153.67 107.95) (width 1) (layer F.Cu) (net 2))
 (segment (start 153.67 107.95) (end 155.829 105.791) (width 1) (layer F.Cu) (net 2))
 (segment (start 127 78.74) (end 127.127 78.867) (width 1) (layer B.Cu) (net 4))
 (segment (start 144.679051 110.49) (end 128.27 110.49) (width 1) (layer B.Cu) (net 4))
 (segment (start 128.27 110.49) (end 124.46 106.68) (width 1) (layer B.Cu) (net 4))
 (segment (start 124.46 106.68) (end 124.46 81.28) (width 1) (layer B.Cu) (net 4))
 (segment (start 127.127 78.867) (end 133.096 78.867) (width 1) (layer B.Cu) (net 4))
 (segment (start 124.46 81.28) (end 127 78.74) (width 1) (layer B.Cu) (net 4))
 (segment (start 144.907 110.262051) (end 144.679051 110.49) (width 1) (layer B.Cu) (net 4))
 (segment (start 144.907 105.537) (end 144.907 110.262051) (width 1) (layer B.Cu) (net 4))
 (segment (start 148.59 111.379) (end 148.59 115.697) (width 1) (layer B.Cu) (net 4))
 (segment (start 144.679051 110.49) (end 147.701 110.49) (width 1) (layer B.Cu) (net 4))
 (segment (start 147.701 110.49) (end 148.59 111.379) (width 1) (layer B.Cu) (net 4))
 (segment (start 105.918 131.016) (end 105.618 131.016) (width 1) (layer B.Cu) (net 12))
 (segment (start 107.468 131.016) (end 108.278 131.826) (width 1) (layer B.Cu) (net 12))
 (segment (start 105.918 131.016) (end 107.468 131.016) (width 1) (layer B.Cu) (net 12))
 (segment (start 171.196 79.89) (end 171.958 80.652) (width 1) (layer B.Cu) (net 12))
 (segment (start 171.196 65.405) (end 171.196 79.89) (width 1) (layer B.Cu) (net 12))
 (segment (start 105.156 104.267) (end 108.077 104.267) (width 1) (layer B.Cu) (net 12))
 (segment (start 108.077 104.267) (end 114.3 110.49) (width 1) (layer B.Cu) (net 12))
 (segment (start 114.3 110.49) (end 114.3 131.826) (width 1) (layer B.Cu) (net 12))
 (segment (start 142.886723 135.358759) (end 142.886723 135.058759) (width 1) (layer B.Cu) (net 12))
 (segment (start 133.477 138.43) (end 142.24 138.43) (width 1) (layer B.Cu) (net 12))
 (segment (start 114.3 131.826) (end 126.873 131.826) (width 1) (layer B.Cu) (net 12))
 (segment (start 135.88 128.407) (end 129.667 134.62) (width 1) (layer B.Cu) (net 12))
 (segment (start 135.88 127) (end 135.88 128.407) (width 1) (layer B.Cu) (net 12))
 (segment (start 126.873 131.826) (end 129.667 134.62) (width 1) (layer B.Cu) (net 12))
 (segment (start 129.667 134.62) (end 133.477 138.43) (width 1) (layer B.Cu) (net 12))
 (segment (start 161.918 80.652) (end 171.958 80.652) (width 1) (layer B.Cu) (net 12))
 (segment (start 160.02 82.55) (end 161.918 80.652) (width 1) (layer B.Cu) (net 12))
 (segment (start 160.02 90.17) (end 160.02 82.55) (width 1) (layer B.Cu) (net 12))
 (segment (start 157.48 124.46) (end 157.48 92.71) (width 1) (layer B.Cu) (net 12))
 (segment (start 157.48 92.71) (end 160.02 90.17) (width 1) (layer B.Cu) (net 12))
 (segment (start 152.4 138.43) (end 153.67 137.16) (width 1) (layer B.Cu) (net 12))
 (segment (start 153.67 137.16) (end 153.67 128.27) (width 1) (layer B.Cu) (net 12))
 (segment (start 153.67 128.27) (end 157.48 124.46) (width 1) (layer B.Cu) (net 12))
 (segment (start 110.617 130.317) (end 110.617 131.826) (width 1) (layer B.Cu) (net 12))
 (segment (start 110.618 130.316) (end 110.617 130.317) (width 1) (layer B.Cu) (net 12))
 (segment (start 110.618 128.016) (end 110.618 130.316) (width 1) (layer B.Cu) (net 12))
 (segment (start 108.278 131.826) (end 110.617 131.826) (width 1) (layer B.Cu) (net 12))
 (segment (start 110.617 131.826) (end 114.3 131.826) (width 1) (layer B.Cu) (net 12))
 (segment (start 152.4 138.43) (end 148.082 138.43) (width 1) (layer B.Cu) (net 12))
 (segment (start 148.082 138.43) (end 148.082 135.001) (width 1) (layer B.Cu) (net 12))
 (segment (start 143.256 137.301) (end 143.256 138.43) (width 1) (layer B.Cu) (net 12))
 (segment (start 143.256 135.001) (end 143.256 137.301) (width 1) (layer B.Cu) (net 12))
 (segment (start 142.24 138.43) (end 143.256 138.43) (width 1) (layer B.Cu) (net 12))
 (segment (start 143.256 138.43) (end 148.082 138.43) (width 1) (layer B.Cu) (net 12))
 (segment (start 172.593 105.474) (end 173.64 106.521) (width 1) (layer B.Cu) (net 10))
 (segment (start 172.593 96.52) (end 172.593 105.474) (width 1) (layer B.Cu) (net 10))
 (segment (start 110.109 111.76) (end 105.156 106.807) (width 1) (layer F.Cu) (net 10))
 (segment (start 142.24 110.49) (end 140.97 111.76) (width 1) (layer F.Cu) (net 10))
 (segment (start 171.45 110.49) (end 142.24 110.49) (width 1) (layer F.Cu) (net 10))
 (segment (start 173.64 106.521) (end 173.64 108.3) (width 1) (layer F.Cu) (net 10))
 (segment (start 173.64 108.3) (end 171.45 110.49) (width 1) (layer F.Cu) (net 10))
 (segment (start 132.08 125.2) (end 137.16 120.12) (width 1) (layer F.Cu) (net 10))
 (segment (start 132.08 127) (end 132.08 125.2) (width 1) (layer F.Cu) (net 10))
 (segment (start 137.16 120.12) (end 137.16 111.76) (width 1) (layer F.Cu) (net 10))
 (segment (start 140.97 111.76) (end 137.16 111.76) (width 1) (layer F.Cu) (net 10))
 (segment (start 137.16 111.76) (end 110.109 111.76) (width 1) (layer F.Cu) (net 10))
 (segment (start 105.156 106.807) (end 109.855 111.506) (width 1) (layer B.Cu) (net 10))
 (segment (start 109.855 111.506) (end 109.855 118.999) (width 1) (layer B.Cu) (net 10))
 (segment (start 105.918 122.936) (end 105.918 125.016) (width 1) (layer B.Cu) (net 10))
 (segment (start 109.855 118.999) (end 105.918 122.936) (width 1) (layer B.Cu) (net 10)))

